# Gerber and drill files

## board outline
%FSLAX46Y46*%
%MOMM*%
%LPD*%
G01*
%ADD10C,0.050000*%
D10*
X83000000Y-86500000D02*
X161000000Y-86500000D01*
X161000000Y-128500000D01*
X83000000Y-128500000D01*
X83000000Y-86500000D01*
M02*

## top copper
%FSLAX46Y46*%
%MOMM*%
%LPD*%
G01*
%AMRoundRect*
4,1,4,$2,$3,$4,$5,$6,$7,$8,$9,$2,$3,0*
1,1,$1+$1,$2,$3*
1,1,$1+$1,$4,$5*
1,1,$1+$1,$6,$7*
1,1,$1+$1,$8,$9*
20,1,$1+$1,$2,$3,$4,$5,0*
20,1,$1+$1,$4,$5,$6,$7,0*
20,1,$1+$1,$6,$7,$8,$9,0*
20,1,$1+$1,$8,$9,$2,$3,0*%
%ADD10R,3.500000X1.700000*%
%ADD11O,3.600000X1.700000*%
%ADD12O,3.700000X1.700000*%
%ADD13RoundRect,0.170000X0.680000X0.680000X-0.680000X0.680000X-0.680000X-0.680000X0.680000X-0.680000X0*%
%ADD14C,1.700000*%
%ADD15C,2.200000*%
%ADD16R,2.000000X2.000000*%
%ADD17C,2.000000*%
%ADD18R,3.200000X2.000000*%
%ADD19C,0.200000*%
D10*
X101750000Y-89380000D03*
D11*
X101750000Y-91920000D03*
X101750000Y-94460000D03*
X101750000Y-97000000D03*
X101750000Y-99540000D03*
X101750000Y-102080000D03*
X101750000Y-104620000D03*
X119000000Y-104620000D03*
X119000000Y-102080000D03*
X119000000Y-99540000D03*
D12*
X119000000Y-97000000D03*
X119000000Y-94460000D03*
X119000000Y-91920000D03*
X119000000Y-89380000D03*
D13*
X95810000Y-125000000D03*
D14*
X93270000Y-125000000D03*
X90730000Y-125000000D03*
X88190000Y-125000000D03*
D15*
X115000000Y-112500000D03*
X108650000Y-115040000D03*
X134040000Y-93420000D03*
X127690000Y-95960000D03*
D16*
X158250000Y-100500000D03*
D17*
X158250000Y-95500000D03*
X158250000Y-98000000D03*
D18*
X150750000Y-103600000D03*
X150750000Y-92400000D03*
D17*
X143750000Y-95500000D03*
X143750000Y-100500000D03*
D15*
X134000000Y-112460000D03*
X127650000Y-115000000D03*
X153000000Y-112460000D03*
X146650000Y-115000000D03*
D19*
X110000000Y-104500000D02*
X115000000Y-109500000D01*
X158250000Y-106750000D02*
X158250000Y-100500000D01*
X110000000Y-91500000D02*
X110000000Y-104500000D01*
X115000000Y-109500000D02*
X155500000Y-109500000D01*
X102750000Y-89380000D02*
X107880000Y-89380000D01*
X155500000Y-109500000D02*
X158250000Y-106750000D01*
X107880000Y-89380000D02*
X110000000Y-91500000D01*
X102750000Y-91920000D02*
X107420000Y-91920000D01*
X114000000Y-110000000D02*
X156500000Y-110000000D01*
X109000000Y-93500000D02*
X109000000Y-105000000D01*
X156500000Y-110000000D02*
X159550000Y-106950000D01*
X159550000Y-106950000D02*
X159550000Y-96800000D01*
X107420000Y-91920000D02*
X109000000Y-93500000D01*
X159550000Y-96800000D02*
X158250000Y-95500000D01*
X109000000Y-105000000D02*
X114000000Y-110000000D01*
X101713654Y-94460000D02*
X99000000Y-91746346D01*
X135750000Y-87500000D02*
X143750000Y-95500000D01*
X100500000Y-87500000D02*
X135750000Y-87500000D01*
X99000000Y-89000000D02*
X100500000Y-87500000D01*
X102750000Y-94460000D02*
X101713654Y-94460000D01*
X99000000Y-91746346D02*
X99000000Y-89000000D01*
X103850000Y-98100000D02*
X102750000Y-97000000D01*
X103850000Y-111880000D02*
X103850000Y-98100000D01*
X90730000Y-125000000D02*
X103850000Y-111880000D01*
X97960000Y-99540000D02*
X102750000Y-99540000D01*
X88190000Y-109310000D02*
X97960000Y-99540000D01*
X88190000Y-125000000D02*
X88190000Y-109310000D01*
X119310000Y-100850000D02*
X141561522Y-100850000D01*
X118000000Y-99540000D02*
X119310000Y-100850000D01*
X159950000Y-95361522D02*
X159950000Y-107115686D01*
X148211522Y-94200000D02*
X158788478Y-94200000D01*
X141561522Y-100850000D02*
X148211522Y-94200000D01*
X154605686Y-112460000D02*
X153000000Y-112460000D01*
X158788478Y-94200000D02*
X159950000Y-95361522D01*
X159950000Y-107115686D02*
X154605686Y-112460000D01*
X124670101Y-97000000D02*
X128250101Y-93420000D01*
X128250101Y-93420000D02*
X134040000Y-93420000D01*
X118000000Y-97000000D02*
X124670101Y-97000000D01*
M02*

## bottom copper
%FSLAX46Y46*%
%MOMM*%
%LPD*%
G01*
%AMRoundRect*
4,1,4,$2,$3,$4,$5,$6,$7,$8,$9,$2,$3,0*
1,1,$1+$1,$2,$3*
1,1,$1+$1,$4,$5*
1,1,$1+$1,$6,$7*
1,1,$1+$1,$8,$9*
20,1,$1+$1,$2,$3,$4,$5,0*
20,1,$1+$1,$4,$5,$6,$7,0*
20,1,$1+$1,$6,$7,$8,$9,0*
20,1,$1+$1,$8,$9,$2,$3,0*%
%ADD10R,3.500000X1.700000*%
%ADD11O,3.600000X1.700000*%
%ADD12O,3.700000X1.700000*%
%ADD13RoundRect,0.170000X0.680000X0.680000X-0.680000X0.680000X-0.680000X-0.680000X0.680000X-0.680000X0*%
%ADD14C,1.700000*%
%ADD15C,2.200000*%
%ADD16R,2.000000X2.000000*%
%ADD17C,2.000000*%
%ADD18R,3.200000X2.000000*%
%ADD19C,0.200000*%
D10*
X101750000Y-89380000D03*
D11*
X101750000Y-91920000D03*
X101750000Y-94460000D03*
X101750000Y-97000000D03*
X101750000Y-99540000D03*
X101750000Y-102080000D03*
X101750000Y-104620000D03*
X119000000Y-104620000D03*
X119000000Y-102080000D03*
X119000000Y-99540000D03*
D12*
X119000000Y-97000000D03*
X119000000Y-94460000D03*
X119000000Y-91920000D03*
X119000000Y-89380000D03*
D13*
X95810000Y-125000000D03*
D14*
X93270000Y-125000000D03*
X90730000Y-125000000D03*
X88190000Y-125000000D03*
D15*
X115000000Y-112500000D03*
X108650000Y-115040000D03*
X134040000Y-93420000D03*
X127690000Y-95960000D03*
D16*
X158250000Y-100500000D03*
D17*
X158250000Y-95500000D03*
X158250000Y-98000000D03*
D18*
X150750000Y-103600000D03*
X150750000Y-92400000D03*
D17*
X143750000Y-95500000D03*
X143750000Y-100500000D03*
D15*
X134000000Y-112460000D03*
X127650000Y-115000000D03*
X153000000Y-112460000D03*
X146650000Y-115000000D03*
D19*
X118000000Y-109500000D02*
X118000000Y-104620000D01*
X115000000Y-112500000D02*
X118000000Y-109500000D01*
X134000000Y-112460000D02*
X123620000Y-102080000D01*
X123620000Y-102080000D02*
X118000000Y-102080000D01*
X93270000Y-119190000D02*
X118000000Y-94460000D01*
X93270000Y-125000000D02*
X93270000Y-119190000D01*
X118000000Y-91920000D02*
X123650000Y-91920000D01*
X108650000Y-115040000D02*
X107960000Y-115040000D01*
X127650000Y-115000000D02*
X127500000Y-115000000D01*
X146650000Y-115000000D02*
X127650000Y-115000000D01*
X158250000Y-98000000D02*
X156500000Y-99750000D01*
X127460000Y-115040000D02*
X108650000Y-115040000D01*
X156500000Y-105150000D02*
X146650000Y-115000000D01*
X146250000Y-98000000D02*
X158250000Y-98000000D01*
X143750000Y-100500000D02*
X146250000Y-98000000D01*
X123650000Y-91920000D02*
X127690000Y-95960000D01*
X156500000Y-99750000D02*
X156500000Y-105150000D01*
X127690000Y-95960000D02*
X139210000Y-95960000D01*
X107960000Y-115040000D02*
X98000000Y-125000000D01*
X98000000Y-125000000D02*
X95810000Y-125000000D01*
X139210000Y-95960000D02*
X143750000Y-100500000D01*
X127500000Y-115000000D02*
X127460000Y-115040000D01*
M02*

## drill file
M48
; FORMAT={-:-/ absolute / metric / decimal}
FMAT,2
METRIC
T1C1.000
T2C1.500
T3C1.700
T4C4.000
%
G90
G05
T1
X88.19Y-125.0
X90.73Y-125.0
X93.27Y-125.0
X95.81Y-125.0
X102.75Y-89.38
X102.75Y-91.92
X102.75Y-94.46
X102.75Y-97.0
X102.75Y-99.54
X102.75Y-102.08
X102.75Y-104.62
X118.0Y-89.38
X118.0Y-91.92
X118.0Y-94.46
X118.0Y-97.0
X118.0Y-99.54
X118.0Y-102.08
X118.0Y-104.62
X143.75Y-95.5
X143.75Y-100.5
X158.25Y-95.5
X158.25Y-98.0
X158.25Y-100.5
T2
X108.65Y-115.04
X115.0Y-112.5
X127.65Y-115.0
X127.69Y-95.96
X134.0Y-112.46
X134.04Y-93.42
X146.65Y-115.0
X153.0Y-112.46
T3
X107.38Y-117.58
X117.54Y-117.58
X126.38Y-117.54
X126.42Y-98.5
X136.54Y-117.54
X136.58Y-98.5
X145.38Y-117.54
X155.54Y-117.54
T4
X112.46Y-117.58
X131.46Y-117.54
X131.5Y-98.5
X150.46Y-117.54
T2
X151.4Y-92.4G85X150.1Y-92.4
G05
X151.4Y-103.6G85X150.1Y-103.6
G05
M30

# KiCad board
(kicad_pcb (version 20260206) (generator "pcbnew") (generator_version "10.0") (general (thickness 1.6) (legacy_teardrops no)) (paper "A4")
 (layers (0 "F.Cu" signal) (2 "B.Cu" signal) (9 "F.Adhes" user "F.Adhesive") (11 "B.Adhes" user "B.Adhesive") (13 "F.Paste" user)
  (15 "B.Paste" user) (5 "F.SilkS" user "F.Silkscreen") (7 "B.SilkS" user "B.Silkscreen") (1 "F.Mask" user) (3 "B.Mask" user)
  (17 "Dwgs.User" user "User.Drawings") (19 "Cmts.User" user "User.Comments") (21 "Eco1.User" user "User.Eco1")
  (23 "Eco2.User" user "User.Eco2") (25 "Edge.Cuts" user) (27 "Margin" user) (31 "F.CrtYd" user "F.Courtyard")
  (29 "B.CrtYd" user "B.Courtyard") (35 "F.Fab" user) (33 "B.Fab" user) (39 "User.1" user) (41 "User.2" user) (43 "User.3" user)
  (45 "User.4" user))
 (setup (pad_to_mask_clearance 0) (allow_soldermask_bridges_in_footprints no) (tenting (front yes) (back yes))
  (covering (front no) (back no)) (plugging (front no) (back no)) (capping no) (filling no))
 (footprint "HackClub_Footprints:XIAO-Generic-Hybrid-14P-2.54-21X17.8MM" (layer "F.Cu") (at 110.375 97)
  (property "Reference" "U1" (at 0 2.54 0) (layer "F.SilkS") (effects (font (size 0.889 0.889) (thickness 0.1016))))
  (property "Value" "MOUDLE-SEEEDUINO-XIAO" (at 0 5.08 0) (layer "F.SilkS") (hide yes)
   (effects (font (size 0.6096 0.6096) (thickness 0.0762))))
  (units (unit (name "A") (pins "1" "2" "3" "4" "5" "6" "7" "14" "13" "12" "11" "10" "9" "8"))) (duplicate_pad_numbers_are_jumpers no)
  (pad "1" thru_hole rect (at -7.625 -7.62) (size 3.5 1.7) (drill 1 (offset -1 0)) (layers "*.Cu" "*.Mask") (remove_unused_layers no)
   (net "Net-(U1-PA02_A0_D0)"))
  (pad "2" thru_hole oval (at -7.625 -5.08) (size 3.6 1.7) (drill 1 (offset -1 0)) (layers "*.Cu" "*.Mask") (remove_unused_layers no)
   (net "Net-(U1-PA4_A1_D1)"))
  (pad "3" thru_hole oval (at -7.625 -2.54) (size 3.6 1.7) (drill 1 (offset -1 0)) (layers "*.Cu" "*.Mask") (remove_unused_layers no)
   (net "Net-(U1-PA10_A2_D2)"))
  (pad "4" thru_hole oval (at -7.625 0) (size 3.6 1.7) (drill 1 (offset -1 0)) (layers "*.Cu" "*.Mask") (remove_unused_layers no)
   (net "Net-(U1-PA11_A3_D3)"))
  (pad "5" thru_hole oval (at -7.625 2.54) (size 3.6 1.7) (drill 1 (offset -1 0)) (layers "*.Cu" "*.Mask") (remove_unused_layers no)
   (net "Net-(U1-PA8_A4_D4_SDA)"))
  (pad "6" thru_hole oval (at -7.625 5.08 180) (size 3.6 1.7) (drill 1 (offset 1 0)) (layers "*.Cu" "*.Mask") (remove_unused_layers no)
   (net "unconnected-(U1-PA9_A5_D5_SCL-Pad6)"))
  (pad "7" thru_hole oval (at -7.625 7.62) (size 3.6 1.7) (drill 1 (offset -1 0)) (layers "*.Cu" "*.Mask") (remove_unused_layers no)
   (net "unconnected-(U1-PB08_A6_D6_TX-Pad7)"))
  (pad "8" thru_hole oval (at 7.625 7.62) (size 3.6 1.7) (drill 1 (offset 1 0)) (layers "*.Cu" "*.Mask") (remove_unused_layers no)
   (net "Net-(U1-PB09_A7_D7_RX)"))
  (pad "9" thru_hole oval (at 7.625 5.08) (size 3.6 1.7) (drill 1 (offset 1 0)) (layers "*.Cu" "*.Mask") (remove_unused_layers no)
   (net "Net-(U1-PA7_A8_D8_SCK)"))
  (pad "10" thru_hole oval (at 7.625 2.54) (size 3.6 1.7) (drill 1 (offset 1 0)) (layers "*.Cu" "*.Mask") (remove_unused_layers no)
   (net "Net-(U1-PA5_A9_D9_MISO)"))
  (pad "11" thru_hole oval (at 7.625 0) (size 3.7 1.7) (drill 1 (offset 1 0)) (layers "*.Cu" "*.Mask") (remove_unused_layers no)
   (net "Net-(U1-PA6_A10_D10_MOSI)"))
  (pad "12" thru_hole oval (at 7.625 -2.54) (size 3.7 1.7) (drill 1 (offset 1 0)) (layers "*.Cu" "*.Mask") (remove_unused_layers no)
   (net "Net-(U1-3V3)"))
  (pad "13" thru_hole oval (at 7.625 -5.08) (size 3.7 1.7) (drill 1 (offset 1 0)) (layers "*.Cu" "*.Mask") (remove_unused_layers no)
   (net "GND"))
  (pad "14" thru_hole oval (at 7.625 -7.62) (size 3.7 1.7) (drill 1 (offset 1 0)) (layers "*.Cu" "*.Mask") (remove_unused_layers no)
   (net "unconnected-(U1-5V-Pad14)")))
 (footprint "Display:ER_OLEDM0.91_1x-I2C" (layer "F.Cu") (at 95.81 125 180)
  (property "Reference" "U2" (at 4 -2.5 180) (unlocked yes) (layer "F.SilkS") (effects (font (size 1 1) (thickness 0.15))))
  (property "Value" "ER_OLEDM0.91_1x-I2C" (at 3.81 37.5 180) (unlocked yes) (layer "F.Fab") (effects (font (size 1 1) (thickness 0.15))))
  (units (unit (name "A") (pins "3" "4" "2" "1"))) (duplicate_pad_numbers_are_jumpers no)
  (pad "1" thru_hole roundrect (at 0 0 180) (size 1.7 1.7) (drill 1) (layers "*.Cu" "*.Mask") (remove_unused_layers no)
   (roundrect_rratio 0.1) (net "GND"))
  (pad "2" thru_hole circle (at 2.54 0 180) (size 1.7 1.7) (drill 1) (layers "*.Cu" "*.Mask") (remove_unused_layers no) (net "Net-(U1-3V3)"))
  (pad "3" thru_hole circle (at 5.08 0 180) (size 1.7 1.7) (drill 1) (layers "*.Cu" "*.Mask") (remove_unused_layers no)
   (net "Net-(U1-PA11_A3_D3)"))
  (pad "4" thru_hole circle (at 7.62 0 180) (size 1.7 1.7) (drill 1) (layers "*.Cu" "*.Mask") (remove_unused_layers no)
   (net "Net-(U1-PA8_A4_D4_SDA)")))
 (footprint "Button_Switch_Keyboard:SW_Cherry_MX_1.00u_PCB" (layer "F.Cu") (at 115 112.5)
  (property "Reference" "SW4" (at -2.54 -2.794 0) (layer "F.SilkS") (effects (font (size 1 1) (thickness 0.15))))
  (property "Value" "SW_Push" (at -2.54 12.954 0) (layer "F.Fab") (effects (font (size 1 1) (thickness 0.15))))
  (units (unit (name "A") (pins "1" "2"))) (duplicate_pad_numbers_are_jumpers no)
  (pad "" np_thru_hole circle (at -7.62 5.08) (size 1.7 1.7) (drill 1.7) (layers "*.Cu" "*.Mask"))
  (pad "" np_thru_hole circle (at -2.54 5.08) (size 4 4) (drill 4) (layers "*.Cu" "*.Mask"))
  (pad "" np_thru_hole circle (at 2.54 5.08) (size 1.7 1.7) (drill 1.7) (layers "*.Cu" "*.Mask"))
  (pad "1" thru_hole circle (at 0 0) (size 2.2 2.2) (drill 1.5) (layers "*.Cu" "*.Mask") (remove_unused_layers no)
   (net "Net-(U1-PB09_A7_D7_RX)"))
  (pad "2" thru_hole circle (at -6.35 2.54) (size 2.2 2.2) (drill 1.5) (layers "*.Cu" "*.Mask") (remove_unused_layers no) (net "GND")))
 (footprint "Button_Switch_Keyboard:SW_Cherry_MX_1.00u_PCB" (layer "F.Cu") (at 134.04 93.42)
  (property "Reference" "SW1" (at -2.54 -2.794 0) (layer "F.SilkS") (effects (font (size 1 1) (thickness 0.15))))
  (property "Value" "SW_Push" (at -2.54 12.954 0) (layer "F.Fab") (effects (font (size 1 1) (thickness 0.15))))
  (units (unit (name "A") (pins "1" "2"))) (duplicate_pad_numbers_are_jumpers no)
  (pad "" np_thru_hole circle (at -7.62 5.08) (size 1.7 1.7) (drill 1.7) (layers "*.Cu" "*.Mask"))
  (pad "" np_thru_hole circle (at -2.54 5.08) (size 4 4) (drill 4) (layers "*.Cu" "*.Mask"))
  (pad "" np_thru_hole circle (at 2.54 5.08) (size 1.7 1.7) (drill 1.7) (layers "*.Cu" "*.Mask"))
  (pad "1" thru_hole circle (at 0 0) (size 2.2 2.2) (drill 1.5) (layers "*.Cu" "*.Mask") (remove_unused_layers no)
   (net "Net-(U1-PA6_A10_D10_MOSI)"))
  (pad "2" thru_hole circle (at -6.35 2.54) (size 2.2 2.2) (drill 1.5) (layers "*.Cu" "*.Mask") (remove_unused_layers no) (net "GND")))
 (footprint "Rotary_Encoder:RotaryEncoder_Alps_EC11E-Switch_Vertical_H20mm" (layer "F.Cu") (at 158.25 100.5 180)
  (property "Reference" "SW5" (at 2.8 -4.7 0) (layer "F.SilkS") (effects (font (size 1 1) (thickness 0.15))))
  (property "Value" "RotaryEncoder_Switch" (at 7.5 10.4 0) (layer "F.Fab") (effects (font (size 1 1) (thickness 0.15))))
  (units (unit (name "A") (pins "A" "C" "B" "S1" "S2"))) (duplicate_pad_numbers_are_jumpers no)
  (pad "A" thru_hole rect (at 0 0 180) (size 2 2) (drill 1) (layers "*.Cu" "*.Mask") (remove_unused_layers no) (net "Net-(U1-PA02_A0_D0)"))
  (pad "B" thru_hole circle (at 0 5 180) (size 2 2) (drill 1) (layers "*.Cu" "*.Mask") (remove_unused_layers no) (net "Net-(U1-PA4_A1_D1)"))
  (pad "C" thru_hole circle (at 0 2.5 180) (size 2 2) (drill 1) (layers "*.Cu" "*.Mask") (remove_unused_layers no) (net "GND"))
  (pad "MP" thru_hole rect (at 7.5 -3.1 180) (size 3.2 2) (drill oval 2.8 1.5) (layers "*.Cu" "*.Mask") (remove_unused_layers no))
  (pad "MP" thru_hole rect (at 7.5 8.1 180) (size 3.2 2) (drill oval 2.8 1.5) (layers "*.Cu" "*.Mask") (remove_unused_layers no))
  (pad "S1" thru_hole circle (at 14.5 5 180) (size 2 2) (drill 1) (layers "*.Cu" "*.Mask") (remove_unused_layers no)
   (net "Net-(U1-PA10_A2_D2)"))
  (pad "S2" thru_hole circle (at 14.5 0 180) (size 2 2) (drill 1) (layers "*.Cu" "*.Mask") (remove_unused_layers no) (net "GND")))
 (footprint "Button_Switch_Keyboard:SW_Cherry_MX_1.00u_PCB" (layer "F.Cu") (at 134 112.46)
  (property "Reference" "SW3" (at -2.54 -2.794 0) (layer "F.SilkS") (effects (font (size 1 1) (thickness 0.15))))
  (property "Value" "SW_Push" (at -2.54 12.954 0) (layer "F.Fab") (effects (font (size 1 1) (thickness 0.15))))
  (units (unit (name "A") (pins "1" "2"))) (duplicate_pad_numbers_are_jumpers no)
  (pad "" np_thru_hole circle (at -7.62 5.08) (size 1.7 1.7) (drill 1.7) (layers "*.Cu" "*.Mask"))
  (pad "" np_thru_hole circle (at -2.54 5.08) (size 4 4) (drill 4) (layers "*.Cu" "*.Mask"))
  (pad "" np_thru_hole circle (at 2.54 5.08) (size 1.7 1.7) (drill 1.7) (layers "*.Cu" "*.Mask"))
  (pad "1" thru_hole circle (at 0 0) (size 2.2 2.2) (drill 1.5) (layers "*.Cu" "*.Mask") (remove_unused_layers no)
   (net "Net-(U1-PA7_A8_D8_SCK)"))
  (pad "2" thru_hole circle (at -6.35 2.54) (size 2.2 2.2) (drill 1.5) (layers "*.Cu" "*.Mask") (remove_unused_layers no) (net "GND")))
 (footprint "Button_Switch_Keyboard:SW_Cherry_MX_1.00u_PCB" (layer "F.Cu") (at 153 112.46)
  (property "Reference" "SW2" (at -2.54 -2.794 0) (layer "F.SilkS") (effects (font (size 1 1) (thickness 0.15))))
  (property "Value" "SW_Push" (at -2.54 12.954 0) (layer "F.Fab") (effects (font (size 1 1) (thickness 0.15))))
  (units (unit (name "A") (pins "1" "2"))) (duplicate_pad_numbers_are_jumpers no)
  (pad "" np_thru_hole circle (at -7.62 5.08) (size 1.7 1.7) (drill 1.7) (layers "*.Cu" "*.Mask"))
  (pad "" np_thru_hole circle (at -2.54 5.08) (size 4 4) (drill 4) (layers "*.Cu" "*.Mask"))
  (pad "" np_thru_hole circle (at 2.54 5.08) (size 1.7 1.7) (drill 1.7) (layers "*.Cu" "*.Mask"))
  (pad "1" thru_hole circle (at 0 0) (size 2.2 2.2) (drill 1.5) (layers "*.Cu" "*.Mask") (remove_unused_layers no)
   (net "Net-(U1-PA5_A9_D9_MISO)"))
  (pad "2" thru_hole circle (at -6.35 2.54) (size 2.2 2.2) (drill 1.5) (layers "*.Cu" "*.Mask") (remove_unused_layers no) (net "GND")))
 (gr_rect (start 83 86.5) (end 161 128.5) (stroke (width 0.05) (type default)) (fill no) (layer "Edge.Cuts"))
 (segment (start 110 104.5) (end 115 109.5) (width 0.2) (layer "F.Cu") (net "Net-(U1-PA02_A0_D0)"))
 (segment (start 158.25 106.75) (end 158.25 100.5) (width 0.2) (layer "F.Cu") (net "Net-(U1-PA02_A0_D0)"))
 (segment (start 110 91.5) (end 110 104.5) (width 0.2) (layer "F.Cu") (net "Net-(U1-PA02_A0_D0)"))
 (segment (start 115 109.5) (end 155.5 109.5) (width 0.2) (layer "F.Cu") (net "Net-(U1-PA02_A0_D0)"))
 (segment (start 102.75 89.38) (end 107.88 89.38) (width 0.2) (layer "F.Cu") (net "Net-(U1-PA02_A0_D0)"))
 (segment (start 155.5 109.5) (end 158.25 106.75) (width 0.2) (layer "F.Cu") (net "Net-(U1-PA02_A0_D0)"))
 (segment (start 107.88 89.38) (end 110 91.5) (width 0.2) (layer "F.Cu") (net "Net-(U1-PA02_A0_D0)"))
 (segment (start 102.75 91.92) (end 107.42 91.92) (width 0.2) (layer "F.Cu") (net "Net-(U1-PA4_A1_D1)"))
 (segment (start 114 110) (end 156.5 110) (width 0.2) (layer "F.Cu") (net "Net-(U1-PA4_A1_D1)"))
 (segment (start 109 93.5) (end 109 105) (width 0.2) (layer "F.Cu") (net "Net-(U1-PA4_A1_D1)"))
 (segment (start 156.5 110) (end 159.55 106.95) (width 0.2) (layer "F.Cu") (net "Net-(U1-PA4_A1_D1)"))
 (segment (start 159.55 106.95) (end 159.55 96.8) (width 0.2) (layer "F.Cu") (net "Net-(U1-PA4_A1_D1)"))
 (segment (start 107.42 91.92) (end 109 93.5) (width 0.2) (layer "F.Cu") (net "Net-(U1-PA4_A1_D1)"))
 (segment (start 159.55 96.8) (end 158.25 95.5) (width 0.2) (layer "F.Cu") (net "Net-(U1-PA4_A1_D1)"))
 (segment (start 109 105) (end 114 110) (width 0.2) (layer "F.Cu") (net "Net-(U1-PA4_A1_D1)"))
 (segment (start 101.713654 94.46) (end 99 91.746346) (width 0.2) (layer "F.Cu") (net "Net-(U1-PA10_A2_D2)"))
 (segment (start 135.75 87.5) (end 143.75 95.5) (width 0.2) (layer "F.Cu") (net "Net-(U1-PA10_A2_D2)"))
 (segment (start 100.5 87.5) (end 135.75 87.5) (width 0.2) (layer "F.Cu") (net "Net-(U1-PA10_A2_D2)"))
 (segment (start 99 89) (end 100.5 87.5) (width 0.2) (layer "F.Cu") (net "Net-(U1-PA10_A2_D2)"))
 (segment (start 102.75 94.46) (end 101.713654 94.46) (width 0.2) (layer "F.Cu") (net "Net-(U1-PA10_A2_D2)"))
 (segment (start 99 91.746346) (end 99 89) (width 0.2) (layer "F.Cu") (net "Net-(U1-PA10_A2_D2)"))
 (segment (start 103.85 98.1) (end 102.75 97) (width 0.2) (layer "F.Cu") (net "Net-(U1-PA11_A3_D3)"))
 (segment (start 103.85 111.88) (end 103.85 98.1) (width 0.2) (layer "F.Cu") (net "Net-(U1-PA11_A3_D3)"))
 (segment (start 90.73 125) (end 103.85 111.88) (width 0.2) (layer "F.Cu") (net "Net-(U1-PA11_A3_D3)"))
 (segment (start 97.96 99.54) (end 102.75 99.54) (width 0.2) (layer "F.Cu") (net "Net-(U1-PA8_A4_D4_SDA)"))
 (segment (start 88.19 109.31) (end 97.96 99.54) (width 0.2) (layer "F.Cu") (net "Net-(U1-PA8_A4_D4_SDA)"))
 (segment (start 88.19 125) (end 88.19 109.31) (width 0.2) (layer "F.Cu") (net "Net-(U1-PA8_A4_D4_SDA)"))
 (segment (start 118 109.5) (end 118 104.62) (width 0.2) (layer "B.Cu") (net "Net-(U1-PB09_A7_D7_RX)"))
 (segment (start 115 112.5) (end 118 109.5) (width 0.2) (layer "B.Cu") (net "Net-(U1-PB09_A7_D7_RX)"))
 (segment (start 134 112.46) (end 123.62 102.08) (width 0.2) (layer "B.Cu") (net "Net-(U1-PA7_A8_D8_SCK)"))
 (segment (start 123.62 102.08) (end 118 102.08) (width 0.2) (layer "B.Cu") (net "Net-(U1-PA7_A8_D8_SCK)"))
 (segment (start 119.31 100.85) (end 141.561522 100.85) (width 0.2) (layer "F.Cu") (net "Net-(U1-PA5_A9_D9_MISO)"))
 (segment (start 118 99.54) (end 119.31 100.85) (width 0.2) (layer "F.Cu") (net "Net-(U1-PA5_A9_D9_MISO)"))
 (segment (start 159.95 95.361522) (end 159.95 107.115686) (width 0.2) (layer "F.Cu") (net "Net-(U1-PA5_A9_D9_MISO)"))
 (segment (start 148.211522 94.2) (end 158.788478 94.2) (width 0.2) (layer "F.Cu") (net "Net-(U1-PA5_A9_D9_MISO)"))
 (segment (start 141.561522 100.85) (end 148.211522 94.2) (width 0.2) (layer "F.Cu") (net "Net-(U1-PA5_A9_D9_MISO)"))
 (segment (start 154.605686 112.46) (end 153 112.46) (width 0.2) (layer "F.Cu") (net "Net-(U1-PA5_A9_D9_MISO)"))
 (segment (start 158.788478 94.2) (end 159.95 95.361522) (width 0.2) (layer "F.Cu") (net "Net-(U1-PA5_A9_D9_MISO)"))
 (segment (start 159.95 107.115686) (end 154.605686 112.46) (width 0.2) (layer "F.Cu") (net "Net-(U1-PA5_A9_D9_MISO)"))
 (segment (start 124.670101 97) (end 128.250101 93.42) (width 0.2) (layer "F.Cu") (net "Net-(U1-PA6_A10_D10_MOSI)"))
 (segment (start 128.250101 93.42) (end 134.04 93.42) (width 0.2) (layer "F.Cu") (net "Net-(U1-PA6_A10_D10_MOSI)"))
 (segment (start 118 97) (end 124.670101 97) (width 0.2) (layer "F.Cu") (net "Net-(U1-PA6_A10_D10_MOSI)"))
 (segment (start 93.27 119.19) (end 118 94.46) (width 0.2) (layer "B.Cu") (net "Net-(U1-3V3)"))
 (segment (start 93.27 125) (end 93.27 119.19) (width 0.2) (layer "B.Cu") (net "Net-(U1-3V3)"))
 (segment (start 118 91.92) (end 123.65 91.92) (width 0.2) (layer "B.Cu") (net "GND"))
 (segment (start 108.65 115.04) (end 107.96 115.04) (width 0.2) (layer "B.Cu") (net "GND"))
 (segment (start 127.65 115) (end 127.5 115) (width 0.2) (layer "B.Cu") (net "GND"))
 (segment (start 146.65 115) (end 127.65 115) (width 0.2) (layer "B.Cu") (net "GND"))
 (segment (start 158.25 98) (end 156.5 99.75) (width 0.2) (layer "B.Cu") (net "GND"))
 (segment (start 127.46 115.04) (end 108.65 115.04) (width 0.2) (layer "B.Cu") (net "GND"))
 (segment (start 156.5 105.15) (end 146.65 115) (width 0.2) (layer "B.Cu") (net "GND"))
 (segment (start 146.25 98) (end 158.25 98) (width 0.2) (layer "B.Cu") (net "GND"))
 (segment (start 143.75 100.5) (end 146.25 98) (width 0.2) (layer "B.Cu") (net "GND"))
 (segment (start 123.65 91.92) (end 127.69 95.96) (width 0.2) (layer "B.Cu") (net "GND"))
 (segment (start 156.5 99.75) (end 156.5 105.15) (width 0.2) (layer "B.Cu") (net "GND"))
 (segment (start 127.69 95.96) (end 139.21 95.96) (width 0.2) (layer "B.Cu") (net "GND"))
 (segment (start 107.96 115.04) (end 98 125) (width 0.2) (layer "B.Cu") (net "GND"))
 (segment (start 98 125) (end 95.81 125) (width 0.2) (layer "B.Cu") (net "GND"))
 (segment (start 139.21 95.96) (end 143.75 100.5) (width 0.2) (layer "B.Cu") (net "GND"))
 (segment (start 127.5 115) (end 127.46 115.04) (width 0.2) (layer "B.Cu") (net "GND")))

